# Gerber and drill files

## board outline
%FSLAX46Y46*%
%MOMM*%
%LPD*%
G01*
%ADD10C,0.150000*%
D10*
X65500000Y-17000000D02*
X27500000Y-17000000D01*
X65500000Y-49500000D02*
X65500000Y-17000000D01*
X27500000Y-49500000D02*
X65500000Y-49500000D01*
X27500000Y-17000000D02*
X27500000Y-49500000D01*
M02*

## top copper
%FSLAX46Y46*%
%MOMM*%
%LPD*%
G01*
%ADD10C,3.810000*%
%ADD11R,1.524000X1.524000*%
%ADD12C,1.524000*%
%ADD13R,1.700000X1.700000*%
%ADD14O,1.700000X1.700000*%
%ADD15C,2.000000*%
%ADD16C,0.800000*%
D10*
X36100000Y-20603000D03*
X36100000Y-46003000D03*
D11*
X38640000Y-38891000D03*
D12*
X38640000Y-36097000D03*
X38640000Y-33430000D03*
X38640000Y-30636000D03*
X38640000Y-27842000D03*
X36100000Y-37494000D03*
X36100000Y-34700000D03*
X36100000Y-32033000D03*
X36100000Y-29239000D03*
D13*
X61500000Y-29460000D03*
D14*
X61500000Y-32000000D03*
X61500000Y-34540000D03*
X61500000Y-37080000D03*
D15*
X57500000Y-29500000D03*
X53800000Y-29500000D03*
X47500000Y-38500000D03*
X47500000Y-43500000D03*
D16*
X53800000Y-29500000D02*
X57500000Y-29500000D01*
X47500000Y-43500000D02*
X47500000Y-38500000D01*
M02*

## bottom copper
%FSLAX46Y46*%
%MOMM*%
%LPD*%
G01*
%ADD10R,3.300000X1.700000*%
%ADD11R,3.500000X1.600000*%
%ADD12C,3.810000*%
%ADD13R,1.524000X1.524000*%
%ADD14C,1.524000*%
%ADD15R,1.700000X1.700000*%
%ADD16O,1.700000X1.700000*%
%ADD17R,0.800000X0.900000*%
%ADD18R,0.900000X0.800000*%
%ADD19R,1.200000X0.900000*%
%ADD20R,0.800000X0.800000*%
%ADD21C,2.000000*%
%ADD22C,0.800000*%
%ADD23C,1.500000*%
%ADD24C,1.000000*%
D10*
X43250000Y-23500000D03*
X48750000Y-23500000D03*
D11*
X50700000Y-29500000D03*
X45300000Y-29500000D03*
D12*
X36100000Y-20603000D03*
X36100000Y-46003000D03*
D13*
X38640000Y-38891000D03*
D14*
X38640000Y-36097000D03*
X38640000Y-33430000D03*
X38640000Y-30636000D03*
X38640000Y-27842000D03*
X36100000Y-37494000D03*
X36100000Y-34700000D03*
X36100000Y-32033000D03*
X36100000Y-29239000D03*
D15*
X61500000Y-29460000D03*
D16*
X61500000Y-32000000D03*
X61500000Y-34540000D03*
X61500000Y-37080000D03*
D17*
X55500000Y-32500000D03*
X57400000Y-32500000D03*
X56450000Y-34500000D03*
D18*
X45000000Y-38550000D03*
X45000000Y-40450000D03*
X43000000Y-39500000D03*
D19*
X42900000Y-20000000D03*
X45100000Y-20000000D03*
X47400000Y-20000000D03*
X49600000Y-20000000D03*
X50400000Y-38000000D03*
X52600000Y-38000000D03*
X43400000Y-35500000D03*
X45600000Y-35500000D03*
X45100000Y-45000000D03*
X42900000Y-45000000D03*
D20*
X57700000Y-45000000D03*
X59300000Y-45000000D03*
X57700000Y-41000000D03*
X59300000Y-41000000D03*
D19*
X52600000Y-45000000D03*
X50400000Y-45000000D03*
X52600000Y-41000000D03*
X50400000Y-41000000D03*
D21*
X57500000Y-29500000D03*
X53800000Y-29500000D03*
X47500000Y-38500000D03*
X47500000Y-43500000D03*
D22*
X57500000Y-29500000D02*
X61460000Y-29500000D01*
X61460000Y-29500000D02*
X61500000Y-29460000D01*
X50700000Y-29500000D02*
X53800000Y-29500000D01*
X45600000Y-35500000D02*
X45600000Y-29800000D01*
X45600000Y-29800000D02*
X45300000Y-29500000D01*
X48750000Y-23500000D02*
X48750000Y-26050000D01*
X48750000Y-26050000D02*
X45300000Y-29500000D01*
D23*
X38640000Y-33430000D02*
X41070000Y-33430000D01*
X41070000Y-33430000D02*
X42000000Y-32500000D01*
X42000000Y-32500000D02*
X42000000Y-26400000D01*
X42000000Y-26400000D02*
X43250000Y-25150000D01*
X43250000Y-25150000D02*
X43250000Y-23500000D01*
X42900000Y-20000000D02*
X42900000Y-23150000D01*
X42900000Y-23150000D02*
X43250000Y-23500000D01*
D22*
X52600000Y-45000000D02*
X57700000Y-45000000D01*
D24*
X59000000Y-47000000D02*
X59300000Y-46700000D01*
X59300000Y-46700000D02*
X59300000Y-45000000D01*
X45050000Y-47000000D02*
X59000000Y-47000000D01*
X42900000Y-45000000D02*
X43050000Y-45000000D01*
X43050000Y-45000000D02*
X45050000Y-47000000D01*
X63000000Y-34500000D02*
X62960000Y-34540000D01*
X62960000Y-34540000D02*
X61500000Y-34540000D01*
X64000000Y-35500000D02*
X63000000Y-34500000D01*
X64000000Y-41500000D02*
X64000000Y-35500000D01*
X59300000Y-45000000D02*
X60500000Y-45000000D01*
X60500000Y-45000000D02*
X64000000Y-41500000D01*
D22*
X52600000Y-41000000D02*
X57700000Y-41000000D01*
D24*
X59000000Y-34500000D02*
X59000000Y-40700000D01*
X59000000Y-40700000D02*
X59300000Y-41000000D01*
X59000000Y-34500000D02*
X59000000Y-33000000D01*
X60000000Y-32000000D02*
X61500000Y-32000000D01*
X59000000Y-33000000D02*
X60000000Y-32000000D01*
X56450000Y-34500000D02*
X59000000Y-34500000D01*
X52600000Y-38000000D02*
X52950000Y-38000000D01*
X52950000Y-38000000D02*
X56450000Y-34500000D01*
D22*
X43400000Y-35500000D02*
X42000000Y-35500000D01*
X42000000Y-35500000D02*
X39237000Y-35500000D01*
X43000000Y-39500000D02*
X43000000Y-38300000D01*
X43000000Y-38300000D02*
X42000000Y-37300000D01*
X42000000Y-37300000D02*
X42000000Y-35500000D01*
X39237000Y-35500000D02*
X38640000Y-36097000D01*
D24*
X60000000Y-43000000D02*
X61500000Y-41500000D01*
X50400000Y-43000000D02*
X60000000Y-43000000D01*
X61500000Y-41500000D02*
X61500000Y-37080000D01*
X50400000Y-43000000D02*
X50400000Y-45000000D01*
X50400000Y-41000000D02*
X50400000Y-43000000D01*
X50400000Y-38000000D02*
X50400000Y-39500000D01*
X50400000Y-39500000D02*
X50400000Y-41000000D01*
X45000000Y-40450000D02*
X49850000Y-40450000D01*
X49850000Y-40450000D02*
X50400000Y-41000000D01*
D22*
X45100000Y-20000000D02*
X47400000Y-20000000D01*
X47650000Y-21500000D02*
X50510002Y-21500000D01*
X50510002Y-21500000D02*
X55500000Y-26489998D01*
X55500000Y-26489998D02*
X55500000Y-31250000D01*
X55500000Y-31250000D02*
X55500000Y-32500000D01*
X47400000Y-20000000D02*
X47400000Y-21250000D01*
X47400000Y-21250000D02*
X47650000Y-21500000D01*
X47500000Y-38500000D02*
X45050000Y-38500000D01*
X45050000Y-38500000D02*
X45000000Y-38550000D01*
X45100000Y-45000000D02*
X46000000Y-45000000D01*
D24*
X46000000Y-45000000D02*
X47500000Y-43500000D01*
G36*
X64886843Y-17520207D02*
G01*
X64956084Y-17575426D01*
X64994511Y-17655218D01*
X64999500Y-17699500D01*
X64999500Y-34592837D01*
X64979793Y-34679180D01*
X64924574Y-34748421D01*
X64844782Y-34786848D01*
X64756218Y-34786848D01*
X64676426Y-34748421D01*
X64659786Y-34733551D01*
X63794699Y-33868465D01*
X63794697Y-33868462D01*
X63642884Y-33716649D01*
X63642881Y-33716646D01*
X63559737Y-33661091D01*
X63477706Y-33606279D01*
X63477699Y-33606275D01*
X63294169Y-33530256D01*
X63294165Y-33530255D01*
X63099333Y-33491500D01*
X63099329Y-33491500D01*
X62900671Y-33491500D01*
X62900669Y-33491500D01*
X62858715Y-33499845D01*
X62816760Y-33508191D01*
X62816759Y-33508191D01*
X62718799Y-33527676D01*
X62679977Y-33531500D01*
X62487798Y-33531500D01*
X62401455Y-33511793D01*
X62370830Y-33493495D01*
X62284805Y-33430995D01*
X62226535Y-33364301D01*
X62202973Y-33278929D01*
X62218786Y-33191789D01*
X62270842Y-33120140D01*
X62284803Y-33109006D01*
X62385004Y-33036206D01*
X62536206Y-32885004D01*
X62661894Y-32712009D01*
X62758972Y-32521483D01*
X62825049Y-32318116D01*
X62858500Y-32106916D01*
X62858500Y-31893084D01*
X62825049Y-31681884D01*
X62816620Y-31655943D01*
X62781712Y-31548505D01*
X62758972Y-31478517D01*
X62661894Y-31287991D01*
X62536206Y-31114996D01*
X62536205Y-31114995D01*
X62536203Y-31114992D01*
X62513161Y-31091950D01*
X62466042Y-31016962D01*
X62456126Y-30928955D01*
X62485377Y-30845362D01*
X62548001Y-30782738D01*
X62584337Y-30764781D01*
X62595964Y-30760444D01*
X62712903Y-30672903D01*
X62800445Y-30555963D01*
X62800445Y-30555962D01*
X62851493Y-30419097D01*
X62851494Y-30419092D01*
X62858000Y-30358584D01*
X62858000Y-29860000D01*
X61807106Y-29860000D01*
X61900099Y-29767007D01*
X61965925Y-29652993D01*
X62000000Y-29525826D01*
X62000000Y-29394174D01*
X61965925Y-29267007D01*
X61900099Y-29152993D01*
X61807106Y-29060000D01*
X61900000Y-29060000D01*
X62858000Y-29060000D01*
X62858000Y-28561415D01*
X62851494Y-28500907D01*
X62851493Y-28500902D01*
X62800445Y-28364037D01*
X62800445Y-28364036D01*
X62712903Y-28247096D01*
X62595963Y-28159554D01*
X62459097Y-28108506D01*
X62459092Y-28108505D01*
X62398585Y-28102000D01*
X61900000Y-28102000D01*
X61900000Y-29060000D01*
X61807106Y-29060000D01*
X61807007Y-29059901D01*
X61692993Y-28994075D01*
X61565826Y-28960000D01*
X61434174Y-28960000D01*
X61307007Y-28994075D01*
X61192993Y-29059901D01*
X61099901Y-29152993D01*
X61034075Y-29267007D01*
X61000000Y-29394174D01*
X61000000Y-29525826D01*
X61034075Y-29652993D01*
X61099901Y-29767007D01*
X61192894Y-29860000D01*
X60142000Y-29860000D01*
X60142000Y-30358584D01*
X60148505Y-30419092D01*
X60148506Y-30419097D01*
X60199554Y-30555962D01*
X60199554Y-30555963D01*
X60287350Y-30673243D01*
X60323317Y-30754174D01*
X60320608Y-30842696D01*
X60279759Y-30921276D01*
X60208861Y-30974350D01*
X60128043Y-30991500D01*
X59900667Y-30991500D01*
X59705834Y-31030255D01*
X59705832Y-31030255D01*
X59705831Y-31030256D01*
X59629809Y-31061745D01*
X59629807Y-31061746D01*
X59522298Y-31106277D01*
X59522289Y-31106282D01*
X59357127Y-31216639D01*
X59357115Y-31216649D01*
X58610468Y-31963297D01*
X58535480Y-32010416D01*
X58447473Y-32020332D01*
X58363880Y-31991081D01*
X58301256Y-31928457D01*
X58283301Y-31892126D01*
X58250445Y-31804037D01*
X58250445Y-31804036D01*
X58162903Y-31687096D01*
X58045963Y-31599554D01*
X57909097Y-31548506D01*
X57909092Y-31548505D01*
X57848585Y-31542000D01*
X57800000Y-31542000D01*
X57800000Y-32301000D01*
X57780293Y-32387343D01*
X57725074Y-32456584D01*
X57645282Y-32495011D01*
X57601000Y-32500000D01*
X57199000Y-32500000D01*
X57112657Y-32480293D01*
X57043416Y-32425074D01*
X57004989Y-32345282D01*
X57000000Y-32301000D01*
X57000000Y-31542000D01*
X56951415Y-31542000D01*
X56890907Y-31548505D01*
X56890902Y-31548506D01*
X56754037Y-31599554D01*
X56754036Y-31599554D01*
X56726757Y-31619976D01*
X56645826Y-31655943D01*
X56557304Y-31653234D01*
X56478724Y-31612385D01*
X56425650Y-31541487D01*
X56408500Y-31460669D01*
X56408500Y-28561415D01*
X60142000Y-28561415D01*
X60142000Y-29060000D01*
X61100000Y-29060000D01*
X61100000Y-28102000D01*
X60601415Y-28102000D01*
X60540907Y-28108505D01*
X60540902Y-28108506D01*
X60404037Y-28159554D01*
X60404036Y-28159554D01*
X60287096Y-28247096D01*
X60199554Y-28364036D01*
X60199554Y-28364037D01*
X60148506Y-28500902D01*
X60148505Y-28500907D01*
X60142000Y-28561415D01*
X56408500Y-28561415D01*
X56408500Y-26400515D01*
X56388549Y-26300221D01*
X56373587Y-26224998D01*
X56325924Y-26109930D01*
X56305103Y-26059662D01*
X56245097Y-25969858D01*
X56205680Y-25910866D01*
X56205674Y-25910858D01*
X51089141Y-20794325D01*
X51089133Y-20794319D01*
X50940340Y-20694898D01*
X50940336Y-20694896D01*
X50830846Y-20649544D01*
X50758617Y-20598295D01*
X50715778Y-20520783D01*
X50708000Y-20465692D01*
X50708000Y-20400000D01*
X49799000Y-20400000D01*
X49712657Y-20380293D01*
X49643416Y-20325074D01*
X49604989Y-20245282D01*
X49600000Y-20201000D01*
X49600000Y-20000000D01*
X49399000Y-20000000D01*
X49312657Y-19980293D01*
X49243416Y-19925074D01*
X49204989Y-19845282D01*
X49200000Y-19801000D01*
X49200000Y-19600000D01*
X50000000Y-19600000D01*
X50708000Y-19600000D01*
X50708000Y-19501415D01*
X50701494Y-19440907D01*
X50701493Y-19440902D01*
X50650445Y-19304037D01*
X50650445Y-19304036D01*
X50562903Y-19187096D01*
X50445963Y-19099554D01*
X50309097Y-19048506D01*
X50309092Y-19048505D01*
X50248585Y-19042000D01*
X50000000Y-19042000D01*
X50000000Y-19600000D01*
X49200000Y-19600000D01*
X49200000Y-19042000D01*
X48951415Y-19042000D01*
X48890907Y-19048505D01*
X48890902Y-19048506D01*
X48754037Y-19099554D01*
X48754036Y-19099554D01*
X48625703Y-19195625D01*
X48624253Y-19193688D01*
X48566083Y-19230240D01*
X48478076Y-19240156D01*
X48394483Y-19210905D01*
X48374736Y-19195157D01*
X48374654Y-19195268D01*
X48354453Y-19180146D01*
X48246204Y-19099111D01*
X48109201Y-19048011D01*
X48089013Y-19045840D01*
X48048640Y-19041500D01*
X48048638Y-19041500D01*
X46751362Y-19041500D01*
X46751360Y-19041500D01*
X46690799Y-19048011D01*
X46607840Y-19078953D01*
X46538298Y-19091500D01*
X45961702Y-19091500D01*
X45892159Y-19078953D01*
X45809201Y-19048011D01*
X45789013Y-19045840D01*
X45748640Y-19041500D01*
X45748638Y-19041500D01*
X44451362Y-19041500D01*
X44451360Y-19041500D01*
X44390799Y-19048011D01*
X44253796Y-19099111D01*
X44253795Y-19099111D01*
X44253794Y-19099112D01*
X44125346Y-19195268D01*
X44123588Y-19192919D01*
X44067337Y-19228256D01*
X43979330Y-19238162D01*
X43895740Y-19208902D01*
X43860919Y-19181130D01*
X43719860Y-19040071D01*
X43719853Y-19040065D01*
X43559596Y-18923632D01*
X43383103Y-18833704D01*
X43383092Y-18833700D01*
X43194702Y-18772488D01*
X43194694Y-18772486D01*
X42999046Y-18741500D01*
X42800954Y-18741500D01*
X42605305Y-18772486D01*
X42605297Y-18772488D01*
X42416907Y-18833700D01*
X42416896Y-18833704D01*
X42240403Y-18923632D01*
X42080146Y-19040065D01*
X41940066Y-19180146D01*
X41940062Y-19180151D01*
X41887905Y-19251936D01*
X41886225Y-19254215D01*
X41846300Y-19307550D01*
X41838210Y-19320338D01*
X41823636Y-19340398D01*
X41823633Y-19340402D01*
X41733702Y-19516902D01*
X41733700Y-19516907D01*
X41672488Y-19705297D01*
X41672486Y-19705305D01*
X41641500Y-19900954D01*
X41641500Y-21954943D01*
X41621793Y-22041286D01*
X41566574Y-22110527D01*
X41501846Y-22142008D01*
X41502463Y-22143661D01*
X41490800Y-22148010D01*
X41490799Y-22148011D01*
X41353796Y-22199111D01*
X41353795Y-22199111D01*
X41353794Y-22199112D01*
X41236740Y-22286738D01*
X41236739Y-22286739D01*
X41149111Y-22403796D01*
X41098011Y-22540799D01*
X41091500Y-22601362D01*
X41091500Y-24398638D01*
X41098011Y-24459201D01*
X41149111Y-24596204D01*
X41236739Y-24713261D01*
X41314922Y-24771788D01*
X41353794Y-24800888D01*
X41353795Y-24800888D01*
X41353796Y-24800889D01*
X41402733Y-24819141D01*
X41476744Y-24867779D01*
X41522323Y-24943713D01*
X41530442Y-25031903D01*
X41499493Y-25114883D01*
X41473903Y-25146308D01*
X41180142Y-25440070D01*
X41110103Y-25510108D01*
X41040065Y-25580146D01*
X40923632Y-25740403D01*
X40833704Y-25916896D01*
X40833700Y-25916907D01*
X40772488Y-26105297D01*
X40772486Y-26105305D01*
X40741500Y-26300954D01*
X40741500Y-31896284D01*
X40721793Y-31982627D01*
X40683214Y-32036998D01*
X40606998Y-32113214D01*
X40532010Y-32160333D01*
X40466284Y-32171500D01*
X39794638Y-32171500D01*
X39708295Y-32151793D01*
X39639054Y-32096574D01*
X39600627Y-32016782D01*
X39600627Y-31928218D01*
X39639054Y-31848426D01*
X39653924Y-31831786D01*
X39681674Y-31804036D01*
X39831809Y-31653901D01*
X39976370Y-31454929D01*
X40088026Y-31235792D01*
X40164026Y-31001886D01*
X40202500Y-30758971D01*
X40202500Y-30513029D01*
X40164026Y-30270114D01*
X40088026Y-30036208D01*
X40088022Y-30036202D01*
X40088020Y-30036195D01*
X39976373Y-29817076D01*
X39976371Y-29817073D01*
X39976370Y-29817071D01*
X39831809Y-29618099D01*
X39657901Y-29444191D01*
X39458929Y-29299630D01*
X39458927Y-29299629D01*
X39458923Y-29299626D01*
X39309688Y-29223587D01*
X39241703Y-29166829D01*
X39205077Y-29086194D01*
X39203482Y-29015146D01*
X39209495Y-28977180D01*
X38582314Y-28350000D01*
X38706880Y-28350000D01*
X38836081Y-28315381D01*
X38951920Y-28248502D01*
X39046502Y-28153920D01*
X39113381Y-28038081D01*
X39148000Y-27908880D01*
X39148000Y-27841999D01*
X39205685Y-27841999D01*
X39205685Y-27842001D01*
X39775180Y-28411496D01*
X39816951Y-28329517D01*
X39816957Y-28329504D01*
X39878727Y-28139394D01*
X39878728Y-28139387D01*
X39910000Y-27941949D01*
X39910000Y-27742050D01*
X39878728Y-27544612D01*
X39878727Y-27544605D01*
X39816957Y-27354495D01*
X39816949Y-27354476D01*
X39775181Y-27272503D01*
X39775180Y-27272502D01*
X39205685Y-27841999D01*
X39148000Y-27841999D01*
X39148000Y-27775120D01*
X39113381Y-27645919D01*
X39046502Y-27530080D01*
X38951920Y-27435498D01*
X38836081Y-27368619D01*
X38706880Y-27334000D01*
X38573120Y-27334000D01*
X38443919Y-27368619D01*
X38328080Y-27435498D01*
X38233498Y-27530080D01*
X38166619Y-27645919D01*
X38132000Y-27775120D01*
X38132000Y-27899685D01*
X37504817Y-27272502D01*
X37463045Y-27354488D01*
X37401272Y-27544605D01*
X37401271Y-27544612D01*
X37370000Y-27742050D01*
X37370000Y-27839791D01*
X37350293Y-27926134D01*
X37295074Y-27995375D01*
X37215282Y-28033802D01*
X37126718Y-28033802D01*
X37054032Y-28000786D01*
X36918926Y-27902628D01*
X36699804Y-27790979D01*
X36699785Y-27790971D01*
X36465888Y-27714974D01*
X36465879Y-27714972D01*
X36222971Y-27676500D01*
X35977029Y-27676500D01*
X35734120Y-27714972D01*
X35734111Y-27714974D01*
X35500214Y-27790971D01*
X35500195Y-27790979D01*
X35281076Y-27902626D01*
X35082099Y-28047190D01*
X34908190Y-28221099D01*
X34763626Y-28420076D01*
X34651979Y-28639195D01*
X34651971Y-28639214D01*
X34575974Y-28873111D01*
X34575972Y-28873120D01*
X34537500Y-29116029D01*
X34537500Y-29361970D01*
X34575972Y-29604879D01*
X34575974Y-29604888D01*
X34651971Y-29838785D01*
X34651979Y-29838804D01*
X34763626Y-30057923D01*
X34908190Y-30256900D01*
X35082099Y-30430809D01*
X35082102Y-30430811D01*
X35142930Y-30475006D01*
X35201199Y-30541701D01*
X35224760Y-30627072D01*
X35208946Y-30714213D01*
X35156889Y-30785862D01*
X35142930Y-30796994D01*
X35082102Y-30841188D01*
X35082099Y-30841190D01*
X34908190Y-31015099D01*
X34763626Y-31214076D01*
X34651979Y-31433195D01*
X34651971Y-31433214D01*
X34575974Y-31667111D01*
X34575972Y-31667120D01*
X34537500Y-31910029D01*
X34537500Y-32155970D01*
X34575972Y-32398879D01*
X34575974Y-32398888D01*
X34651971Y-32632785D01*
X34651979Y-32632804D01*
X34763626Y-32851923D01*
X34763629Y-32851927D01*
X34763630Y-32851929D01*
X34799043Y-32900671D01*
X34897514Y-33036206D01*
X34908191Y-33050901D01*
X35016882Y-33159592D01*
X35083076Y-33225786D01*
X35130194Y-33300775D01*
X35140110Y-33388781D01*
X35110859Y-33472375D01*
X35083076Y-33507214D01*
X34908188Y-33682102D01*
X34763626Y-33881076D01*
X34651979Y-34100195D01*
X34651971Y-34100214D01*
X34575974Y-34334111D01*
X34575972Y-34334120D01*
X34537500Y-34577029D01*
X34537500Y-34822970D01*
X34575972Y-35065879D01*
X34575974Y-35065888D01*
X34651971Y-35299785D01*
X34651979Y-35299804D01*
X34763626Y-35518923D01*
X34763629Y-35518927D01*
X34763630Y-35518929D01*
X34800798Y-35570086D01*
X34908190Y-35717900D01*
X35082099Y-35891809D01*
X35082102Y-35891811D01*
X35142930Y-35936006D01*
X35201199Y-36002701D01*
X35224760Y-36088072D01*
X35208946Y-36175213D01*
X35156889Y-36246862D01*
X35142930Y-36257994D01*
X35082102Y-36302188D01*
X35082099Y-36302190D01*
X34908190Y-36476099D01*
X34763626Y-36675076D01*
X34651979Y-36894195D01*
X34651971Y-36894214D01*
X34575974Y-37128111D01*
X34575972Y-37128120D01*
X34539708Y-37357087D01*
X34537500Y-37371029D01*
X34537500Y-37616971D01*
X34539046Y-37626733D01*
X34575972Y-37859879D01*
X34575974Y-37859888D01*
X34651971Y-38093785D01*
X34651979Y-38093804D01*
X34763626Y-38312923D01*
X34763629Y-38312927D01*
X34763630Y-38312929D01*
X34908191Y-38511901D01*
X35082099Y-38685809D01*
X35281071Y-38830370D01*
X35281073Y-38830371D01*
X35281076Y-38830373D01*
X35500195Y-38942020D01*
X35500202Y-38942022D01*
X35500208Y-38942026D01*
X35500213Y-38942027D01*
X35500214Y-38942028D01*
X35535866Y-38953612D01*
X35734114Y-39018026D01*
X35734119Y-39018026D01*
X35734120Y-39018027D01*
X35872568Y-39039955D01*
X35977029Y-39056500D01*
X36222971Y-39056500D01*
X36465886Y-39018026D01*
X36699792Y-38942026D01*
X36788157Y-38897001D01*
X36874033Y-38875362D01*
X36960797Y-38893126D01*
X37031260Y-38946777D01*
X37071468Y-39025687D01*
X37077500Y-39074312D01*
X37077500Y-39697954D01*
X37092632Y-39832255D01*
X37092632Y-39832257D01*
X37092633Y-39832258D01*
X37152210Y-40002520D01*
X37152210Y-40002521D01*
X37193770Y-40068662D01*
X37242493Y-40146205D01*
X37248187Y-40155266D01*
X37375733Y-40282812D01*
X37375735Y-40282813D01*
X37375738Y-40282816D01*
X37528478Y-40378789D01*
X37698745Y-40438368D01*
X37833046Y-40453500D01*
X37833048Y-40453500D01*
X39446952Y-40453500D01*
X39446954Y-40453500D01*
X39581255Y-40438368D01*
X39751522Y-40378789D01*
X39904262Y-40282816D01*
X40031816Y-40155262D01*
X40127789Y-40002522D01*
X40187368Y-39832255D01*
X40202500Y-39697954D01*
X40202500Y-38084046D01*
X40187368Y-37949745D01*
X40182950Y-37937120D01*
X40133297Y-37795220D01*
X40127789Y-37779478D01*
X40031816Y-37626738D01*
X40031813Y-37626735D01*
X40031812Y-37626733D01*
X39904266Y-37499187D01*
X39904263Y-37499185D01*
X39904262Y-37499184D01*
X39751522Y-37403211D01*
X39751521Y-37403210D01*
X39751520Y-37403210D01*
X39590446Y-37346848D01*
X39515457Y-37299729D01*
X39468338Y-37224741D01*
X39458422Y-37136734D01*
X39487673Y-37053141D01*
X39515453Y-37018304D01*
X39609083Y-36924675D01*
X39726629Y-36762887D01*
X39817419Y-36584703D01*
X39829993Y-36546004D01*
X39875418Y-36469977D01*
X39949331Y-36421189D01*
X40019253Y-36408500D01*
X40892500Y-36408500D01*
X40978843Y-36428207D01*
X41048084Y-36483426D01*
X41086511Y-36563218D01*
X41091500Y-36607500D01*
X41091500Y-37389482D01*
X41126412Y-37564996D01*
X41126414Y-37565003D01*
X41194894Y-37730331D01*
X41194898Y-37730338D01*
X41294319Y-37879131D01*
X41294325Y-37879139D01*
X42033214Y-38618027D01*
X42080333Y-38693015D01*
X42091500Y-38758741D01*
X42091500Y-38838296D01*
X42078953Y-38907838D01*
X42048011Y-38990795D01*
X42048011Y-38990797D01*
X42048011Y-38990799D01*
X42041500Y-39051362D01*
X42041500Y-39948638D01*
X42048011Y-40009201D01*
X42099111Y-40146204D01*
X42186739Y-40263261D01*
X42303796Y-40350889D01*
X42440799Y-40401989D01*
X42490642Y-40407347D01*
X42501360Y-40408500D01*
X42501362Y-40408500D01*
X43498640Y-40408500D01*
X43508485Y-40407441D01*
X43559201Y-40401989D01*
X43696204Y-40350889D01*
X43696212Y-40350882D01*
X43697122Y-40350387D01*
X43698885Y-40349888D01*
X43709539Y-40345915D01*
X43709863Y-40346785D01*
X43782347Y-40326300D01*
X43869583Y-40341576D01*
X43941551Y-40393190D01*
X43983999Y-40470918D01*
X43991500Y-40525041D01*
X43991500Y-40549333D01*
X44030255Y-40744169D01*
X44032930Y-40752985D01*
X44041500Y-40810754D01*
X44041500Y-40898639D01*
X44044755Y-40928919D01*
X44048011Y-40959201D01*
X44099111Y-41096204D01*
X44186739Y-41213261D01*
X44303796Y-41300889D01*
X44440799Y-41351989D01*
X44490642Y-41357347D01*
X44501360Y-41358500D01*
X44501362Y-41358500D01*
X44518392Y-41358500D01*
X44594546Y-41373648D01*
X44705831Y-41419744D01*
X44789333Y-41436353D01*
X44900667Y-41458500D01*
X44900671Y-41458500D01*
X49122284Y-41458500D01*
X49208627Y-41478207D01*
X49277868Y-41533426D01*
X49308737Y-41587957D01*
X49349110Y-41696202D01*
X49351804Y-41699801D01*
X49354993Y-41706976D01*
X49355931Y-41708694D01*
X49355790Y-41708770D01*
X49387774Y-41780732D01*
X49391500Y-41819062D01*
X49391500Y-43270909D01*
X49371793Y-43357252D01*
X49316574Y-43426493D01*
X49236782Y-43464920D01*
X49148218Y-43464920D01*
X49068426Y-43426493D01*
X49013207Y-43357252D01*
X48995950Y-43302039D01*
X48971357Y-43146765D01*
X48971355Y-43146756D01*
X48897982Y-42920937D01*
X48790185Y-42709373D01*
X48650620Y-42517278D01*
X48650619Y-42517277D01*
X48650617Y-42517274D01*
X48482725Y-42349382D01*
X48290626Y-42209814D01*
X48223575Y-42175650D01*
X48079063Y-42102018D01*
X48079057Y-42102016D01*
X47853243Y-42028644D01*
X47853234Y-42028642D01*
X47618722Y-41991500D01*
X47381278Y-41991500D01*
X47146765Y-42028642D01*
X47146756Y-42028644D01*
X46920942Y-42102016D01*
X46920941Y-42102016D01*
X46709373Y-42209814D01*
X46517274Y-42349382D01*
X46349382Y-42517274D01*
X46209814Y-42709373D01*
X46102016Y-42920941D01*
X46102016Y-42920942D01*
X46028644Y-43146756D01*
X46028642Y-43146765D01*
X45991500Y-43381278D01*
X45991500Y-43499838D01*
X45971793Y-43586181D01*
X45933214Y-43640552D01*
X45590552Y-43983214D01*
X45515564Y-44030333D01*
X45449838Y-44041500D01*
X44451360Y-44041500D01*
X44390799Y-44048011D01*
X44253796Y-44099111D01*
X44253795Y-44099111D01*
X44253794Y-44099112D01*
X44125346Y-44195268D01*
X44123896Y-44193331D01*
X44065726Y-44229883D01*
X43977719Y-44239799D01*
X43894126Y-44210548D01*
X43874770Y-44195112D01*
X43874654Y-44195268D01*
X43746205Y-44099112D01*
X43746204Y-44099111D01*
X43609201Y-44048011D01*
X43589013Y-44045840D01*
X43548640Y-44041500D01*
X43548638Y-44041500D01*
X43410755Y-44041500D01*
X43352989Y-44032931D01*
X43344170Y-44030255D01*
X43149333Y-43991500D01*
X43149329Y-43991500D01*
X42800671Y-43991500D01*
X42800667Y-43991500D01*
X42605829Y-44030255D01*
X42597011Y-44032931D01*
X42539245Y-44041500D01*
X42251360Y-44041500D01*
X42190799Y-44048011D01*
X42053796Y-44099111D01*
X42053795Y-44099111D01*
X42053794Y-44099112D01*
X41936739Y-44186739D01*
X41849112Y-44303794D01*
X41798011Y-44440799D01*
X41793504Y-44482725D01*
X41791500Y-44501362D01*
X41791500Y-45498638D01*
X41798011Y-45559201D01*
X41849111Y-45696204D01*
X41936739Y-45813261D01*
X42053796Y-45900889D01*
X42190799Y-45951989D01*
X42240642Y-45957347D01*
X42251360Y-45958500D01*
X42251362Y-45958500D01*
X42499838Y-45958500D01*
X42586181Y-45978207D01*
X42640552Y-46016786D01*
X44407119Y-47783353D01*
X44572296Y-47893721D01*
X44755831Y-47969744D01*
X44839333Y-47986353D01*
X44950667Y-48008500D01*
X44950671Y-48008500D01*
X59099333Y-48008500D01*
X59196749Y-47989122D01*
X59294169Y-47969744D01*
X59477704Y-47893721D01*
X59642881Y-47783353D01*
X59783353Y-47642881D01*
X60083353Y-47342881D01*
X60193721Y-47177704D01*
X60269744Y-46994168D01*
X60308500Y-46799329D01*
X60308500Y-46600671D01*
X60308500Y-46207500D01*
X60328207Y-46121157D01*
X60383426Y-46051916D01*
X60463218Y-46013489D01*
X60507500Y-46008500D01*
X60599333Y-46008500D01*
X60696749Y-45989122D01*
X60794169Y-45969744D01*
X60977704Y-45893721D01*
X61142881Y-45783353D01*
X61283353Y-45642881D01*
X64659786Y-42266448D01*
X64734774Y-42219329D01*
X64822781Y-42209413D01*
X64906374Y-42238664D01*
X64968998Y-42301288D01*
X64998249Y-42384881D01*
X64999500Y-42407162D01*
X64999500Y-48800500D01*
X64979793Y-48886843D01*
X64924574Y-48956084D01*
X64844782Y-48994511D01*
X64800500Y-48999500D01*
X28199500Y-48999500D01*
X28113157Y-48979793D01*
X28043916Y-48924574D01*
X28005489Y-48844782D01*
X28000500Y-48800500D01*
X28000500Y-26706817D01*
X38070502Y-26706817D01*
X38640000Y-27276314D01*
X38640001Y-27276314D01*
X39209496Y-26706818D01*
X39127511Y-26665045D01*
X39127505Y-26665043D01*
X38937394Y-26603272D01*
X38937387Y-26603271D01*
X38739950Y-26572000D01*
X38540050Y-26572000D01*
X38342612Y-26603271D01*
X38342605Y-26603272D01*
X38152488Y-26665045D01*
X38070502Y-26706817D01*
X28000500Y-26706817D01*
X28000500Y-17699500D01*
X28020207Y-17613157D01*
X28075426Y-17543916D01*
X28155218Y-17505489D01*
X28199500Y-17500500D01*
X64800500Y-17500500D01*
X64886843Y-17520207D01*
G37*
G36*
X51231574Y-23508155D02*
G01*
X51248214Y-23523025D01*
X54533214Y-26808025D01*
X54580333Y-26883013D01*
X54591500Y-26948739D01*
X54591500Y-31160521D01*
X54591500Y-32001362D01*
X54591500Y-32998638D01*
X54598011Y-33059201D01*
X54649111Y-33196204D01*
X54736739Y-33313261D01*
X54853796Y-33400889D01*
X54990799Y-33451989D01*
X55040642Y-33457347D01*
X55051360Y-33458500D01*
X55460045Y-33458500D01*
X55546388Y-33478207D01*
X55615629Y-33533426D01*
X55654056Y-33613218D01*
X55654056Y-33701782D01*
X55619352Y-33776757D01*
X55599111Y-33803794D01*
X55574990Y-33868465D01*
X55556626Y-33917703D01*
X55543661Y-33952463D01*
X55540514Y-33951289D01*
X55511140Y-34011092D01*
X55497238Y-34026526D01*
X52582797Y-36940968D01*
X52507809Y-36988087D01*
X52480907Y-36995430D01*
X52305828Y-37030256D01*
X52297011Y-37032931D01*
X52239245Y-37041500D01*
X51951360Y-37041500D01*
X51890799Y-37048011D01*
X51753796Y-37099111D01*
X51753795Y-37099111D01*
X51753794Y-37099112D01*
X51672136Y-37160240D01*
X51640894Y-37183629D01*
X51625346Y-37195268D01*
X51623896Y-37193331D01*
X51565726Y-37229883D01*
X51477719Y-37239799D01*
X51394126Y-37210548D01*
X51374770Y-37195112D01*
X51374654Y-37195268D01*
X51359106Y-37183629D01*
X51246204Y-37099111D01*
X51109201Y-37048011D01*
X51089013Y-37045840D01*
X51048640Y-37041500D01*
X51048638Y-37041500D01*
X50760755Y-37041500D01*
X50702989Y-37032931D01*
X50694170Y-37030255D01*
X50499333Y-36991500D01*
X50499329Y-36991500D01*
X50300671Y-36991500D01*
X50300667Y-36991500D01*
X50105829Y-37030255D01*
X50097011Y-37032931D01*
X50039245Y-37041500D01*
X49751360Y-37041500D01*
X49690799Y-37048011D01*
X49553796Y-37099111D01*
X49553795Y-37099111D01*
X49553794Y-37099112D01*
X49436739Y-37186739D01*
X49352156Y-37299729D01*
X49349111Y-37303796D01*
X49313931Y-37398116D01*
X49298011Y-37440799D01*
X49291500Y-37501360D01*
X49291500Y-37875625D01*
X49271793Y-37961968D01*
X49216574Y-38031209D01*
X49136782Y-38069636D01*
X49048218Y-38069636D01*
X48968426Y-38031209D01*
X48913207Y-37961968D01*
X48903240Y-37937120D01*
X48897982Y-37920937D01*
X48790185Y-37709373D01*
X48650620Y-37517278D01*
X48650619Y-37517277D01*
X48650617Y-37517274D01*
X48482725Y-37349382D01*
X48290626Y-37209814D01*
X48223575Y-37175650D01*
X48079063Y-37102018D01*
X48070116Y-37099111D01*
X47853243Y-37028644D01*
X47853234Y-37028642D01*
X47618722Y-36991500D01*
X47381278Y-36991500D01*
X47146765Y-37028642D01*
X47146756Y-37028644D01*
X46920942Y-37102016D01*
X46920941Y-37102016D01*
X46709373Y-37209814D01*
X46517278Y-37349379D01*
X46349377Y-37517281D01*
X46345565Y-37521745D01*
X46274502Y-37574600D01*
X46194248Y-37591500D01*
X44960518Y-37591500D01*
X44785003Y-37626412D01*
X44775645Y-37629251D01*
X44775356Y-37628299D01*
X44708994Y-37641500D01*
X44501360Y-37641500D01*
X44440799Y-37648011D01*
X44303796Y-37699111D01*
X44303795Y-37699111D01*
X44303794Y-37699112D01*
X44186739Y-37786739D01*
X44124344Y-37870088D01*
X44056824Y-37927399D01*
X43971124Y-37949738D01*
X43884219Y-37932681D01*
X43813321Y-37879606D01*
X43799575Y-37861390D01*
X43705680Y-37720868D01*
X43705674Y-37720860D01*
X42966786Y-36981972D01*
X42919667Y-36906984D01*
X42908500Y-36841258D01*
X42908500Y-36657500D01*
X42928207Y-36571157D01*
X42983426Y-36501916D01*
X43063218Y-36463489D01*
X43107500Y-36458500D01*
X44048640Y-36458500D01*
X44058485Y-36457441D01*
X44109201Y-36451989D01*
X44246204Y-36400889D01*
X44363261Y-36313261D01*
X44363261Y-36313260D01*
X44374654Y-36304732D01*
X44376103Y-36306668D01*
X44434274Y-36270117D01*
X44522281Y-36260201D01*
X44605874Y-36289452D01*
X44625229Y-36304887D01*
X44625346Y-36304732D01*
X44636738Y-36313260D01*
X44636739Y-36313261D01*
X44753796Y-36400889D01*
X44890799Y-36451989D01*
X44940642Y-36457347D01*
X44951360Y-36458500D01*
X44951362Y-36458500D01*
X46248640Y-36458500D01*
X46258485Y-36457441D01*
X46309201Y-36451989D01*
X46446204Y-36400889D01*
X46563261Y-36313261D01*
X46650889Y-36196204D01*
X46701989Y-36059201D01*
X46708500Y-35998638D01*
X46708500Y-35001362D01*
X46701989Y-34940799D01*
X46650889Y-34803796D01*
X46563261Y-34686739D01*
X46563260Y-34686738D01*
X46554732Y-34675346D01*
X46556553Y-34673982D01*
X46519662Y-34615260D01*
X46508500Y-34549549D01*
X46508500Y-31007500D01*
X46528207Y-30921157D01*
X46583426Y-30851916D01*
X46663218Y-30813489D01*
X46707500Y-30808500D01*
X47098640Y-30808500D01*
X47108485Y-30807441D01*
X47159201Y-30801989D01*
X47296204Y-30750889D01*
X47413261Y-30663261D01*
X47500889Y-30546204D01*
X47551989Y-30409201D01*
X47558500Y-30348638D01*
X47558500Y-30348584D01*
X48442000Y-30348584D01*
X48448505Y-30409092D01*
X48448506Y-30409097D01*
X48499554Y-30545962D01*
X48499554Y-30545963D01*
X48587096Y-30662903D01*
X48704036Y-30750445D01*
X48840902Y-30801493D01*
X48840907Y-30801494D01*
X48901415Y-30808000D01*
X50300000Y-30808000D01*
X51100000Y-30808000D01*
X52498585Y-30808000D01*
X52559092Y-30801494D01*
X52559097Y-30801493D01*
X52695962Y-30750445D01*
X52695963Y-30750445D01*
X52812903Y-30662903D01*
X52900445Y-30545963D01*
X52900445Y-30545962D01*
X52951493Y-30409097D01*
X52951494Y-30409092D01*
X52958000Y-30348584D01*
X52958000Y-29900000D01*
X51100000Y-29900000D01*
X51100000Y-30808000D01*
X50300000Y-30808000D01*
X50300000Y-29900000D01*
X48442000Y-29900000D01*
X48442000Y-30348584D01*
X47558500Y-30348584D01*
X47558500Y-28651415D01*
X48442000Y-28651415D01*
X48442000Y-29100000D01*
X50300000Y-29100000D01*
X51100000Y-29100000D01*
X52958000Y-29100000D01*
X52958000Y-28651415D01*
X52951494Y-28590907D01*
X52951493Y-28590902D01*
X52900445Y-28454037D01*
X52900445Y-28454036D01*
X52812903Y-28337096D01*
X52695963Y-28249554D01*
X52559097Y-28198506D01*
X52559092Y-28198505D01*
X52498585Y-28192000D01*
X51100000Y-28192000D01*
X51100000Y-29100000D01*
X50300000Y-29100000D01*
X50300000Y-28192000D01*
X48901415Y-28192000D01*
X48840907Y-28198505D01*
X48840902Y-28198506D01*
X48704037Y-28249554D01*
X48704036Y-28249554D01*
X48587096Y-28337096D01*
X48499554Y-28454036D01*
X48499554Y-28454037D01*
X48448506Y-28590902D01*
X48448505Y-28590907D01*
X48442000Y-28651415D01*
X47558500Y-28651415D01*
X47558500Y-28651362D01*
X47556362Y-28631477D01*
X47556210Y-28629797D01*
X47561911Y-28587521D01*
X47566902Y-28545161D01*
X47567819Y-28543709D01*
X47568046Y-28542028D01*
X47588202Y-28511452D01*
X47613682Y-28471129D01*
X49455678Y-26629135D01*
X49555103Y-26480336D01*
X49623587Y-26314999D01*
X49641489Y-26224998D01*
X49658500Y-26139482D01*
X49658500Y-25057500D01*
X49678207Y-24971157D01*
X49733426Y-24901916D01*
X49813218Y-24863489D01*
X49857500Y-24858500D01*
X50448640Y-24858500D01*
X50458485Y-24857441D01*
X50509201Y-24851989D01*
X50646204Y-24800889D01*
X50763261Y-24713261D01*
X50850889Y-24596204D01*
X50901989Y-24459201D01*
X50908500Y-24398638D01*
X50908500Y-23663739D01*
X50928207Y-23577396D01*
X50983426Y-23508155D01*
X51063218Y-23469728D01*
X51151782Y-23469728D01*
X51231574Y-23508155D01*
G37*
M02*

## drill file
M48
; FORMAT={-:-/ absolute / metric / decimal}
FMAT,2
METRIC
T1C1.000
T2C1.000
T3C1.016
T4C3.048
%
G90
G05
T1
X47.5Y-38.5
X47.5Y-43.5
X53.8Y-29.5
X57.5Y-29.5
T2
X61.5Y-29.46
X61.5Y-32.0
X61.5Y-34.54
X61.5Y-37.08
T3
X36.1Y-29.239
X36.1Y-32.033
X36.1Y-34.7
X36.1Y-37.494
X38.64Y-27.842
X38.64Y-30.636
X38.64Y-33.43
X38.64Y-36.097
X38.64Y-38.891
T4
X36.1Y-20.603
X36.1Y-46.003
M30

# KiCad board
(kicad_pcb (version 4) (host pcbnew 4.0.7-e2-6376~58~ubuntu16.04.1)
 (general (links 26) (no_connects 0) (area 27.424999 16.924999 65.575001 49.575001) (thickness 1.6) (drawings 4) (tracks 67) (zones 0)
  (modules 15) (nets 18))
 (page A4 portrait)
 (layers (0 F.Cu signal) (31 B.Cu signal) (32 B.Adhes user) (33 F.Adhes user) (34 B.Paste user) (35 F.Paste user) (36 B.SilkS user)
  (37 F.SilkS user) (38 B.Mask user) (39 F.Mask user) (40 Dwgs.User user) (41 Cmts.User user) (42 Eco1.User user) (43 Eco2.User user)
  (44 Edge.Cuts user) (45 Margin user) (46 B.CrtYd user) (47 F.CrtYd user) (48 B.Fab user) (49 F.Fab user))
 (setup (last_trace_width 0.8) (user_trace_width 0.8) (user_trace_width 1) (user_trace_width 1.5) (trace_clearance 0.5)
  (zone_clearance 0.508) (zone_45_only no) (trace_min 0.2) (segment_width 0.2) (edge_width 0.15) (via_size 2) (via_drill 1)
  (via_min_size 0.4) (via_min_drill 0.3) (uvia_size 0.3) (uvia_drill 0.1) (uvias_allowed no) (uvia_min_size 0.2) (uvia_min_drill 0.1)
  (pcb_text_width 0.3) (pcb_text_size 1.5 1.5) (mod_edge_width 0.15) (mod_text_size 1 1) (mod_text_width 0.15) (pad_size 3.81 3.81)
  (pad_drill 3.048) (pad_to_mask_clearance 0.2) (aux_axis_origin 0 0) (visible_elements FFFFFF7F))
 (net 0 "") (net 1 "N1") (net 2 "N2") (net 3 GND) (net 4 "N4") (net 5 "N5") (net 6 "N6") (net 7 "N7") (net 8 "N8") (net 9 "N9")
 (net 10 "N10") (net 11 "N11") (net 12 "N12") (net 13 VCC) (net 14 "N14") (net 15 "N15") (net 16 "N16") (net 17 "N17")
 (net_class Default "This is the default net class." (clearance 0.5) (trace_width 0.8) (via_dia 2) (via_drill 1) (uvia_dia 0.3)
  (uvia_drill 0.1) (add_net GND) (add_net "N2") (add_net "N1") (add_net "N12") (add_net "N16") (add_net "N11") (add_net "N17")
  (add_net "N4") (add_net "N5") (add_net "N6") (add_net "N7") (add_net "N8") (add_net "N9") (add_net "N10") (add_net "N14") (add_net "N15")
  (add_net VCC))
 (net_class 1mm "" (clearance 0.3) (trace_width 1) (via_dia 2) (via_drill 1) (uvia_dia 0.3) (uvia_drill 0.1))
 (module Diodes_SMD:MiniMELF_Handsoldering (layer B.Cu) (at 46 23.5)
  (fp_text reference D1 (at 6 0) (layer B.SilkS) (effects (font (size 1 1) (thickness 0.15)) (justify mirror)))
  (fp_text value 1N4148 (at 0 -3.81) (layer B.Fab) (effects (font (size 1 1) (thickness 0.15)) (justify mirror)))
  (pad 1 smd rect (at -2.75 0) (size 3.3 1.7) (layers B.Cu B.Paste B.Mask) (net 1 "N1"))
  (pad 2 smd rect (at 2.75 0) (size 3.3 1.7) (layers B.Cu B.Paste B.Mask) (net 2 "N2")))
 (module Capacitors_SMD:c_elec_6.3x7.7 (layer B.Cu) (at 48 29.5 180)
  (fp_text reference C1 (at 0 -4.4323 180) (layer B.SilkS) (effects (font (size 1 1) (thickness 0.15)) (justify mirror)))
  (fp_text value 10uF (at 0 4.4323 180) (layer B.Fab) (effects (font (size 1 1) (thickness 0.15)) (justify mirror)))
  (pad 1 smd rect (at -2.7 0) (size 3.5 1.6) (layers B.Cu B.Paste B.Mask) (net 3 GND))
  (pad 2 smd rect (at 2.7 0) (size 3.5 1.6) (layers B.Cu B.Paste B.Mask) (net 2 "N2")))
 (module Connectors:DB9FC (layer F.Cu) (at 37.37 33.43 90)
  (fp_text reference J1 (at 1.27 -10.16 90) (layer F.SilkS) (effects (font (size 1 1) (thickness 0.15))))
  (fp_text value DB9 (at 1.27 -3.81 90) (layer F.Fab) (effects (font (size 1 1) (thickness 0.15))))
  (pad "" thru_hole circle (at 12.827 -1.27 90) (size 3.81 3.81) (drill 3.048) (layers *.Cu *.Mask) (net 3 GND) (zone_connect 2))
  (pad "" thru_hole circle (at -12.573 -1.27 90) (size 3.81 3.81) (drill 3.048) (layers *.Cu *.Mask) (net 3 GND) (zone_connect 2))
  (pad 1 thru_hole rect (at -5.461 1.27 90) (size 1.524 1.524) (drill 1.016) (layers *.Cu *.Mask) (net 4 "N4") (clearance 0.8))
  (pad 2 thru_hole circle (at -2.667 1.27 90) (size 1.524 1.524) (drill 1.016) (layers *.Cu *.Mask) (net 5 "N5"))
  (pad 3 thru_hole circle (at 0 1.27 90) (size 1.524 1.524) (drill 1.016) (layers *.Cu *.Mask) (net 1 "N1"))
  (pad 4 thru_hole circle (at 2.794 1.27 90) (size 1.524 1.524) (drill 1.016) (layers *.Cu *.Mask) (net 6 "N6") (clearance 0.8))
  (pad 5 thru_hole circle (at 5.588 1.27 90) (size 1.524 1.524) (drill 1.016) (layers *.Cu *.Mask) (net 3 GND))
  (pad 6 thru_hole circle (at -4.064 -1.27 90) (size 1.524 1.524) (drill 1.016) (layers *.Cu *.Mask) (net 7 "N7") (clearance 0.8))
  (pad 7 thru_hole circle (at -1.27 -1.27 90) (size 1.524 1.524) (drill 1.016) (layers *.Cu *.Mask) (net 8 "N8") (clearance 0.8))
  (pad 8 thru_hole circle (at 1.397 -1.27 90) (size 1.524 1.524) (drill 1.016) (layers *.Cu *.Mask) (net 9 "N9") (clearance 0.8))
  (pad 9 thru_hole circle (at 4.191 -1.27 90) (size 1.524 1.524) (drill 1.016) (layers *.Cu *.Mask) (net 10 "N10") (clearance 0.8)))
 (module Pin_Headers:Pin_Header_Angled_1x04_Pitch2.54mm (layer F.Cu) (at 61.5 29.46)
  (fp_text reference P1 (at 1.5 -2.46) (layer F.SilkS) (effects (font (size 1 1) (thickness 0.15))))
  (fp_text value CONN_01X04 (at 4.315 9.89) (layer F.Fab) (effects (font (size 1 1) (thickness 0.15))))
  (pad 1 thru_hole rect (at 0 0) (size 1.7 1.7) (drill 1) (layers *.Cu *.Mask) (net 3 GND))
  (pad 2 thru_hole oval (at 0 2.54) (size 1.7 1.7) (drill 1) (layers *.Cu *.Mask) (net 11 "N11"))
  (pad 3 thru_hole oval (at 0 5.08) (size 1.7 1.7) (drill 1) (layers *.Cu *.Mask) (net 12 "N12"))
  (pad 4 thru_hole oval (at 0 7.62) (size 1.7 1.7) (drill 1) (layers *.Cu *.Mask) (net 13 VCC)))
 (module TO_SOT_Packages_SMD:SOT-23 (layer B.Cu) (at 56.45 33.5 270)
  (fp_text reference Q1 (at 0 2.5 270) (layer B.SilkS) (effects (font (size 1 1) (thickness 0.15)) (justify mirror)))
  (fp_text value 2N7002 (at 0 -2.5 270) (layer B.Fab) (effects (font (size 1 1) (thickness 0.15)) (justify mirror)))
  (pad 1 smd rect (at -1 0.95 270) (size 0.9 0.8) (layers B.Cu B.Paste B.Mask) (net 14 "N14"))
  (pad 2 smd rect (at -1 -0.95 270) (size 0.9 0.8) (layers B.Cu B.Paste B.Mask) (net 3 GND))
  (pad 3 smd rect (at 1 0 270) (size 0.9 0.8) (layers B.Cu B.Paste B.Mask) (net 11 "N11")))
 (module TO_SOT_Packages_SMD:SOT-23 (layer B.Cu) (at 44 39.5 180)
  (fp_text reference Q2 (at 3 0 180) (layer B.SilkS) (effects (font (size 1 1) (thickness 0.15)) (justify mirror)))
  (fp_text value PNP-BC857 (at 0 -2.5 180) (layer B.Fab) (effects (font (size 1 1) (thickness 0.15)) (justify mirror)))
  (pad 1 smd rect (at -1 0.95 180) (size 0.9 0.8) (layers B.Cu B.Paste B.Mask) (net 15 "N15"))
  (pad 2 smd rect (at -1 -0.95 180) (size 0.9 0.8) (layers B.Cu B.Paste B.Mask) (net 13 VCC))
  (pad 3 smd rect (at 1 0 180) (size 0.9 0.8) (layers B.Cu B.Paste B.Mask) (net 5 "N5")))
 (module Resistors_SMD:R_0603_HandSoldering (layer B.Cu) (at 44 20)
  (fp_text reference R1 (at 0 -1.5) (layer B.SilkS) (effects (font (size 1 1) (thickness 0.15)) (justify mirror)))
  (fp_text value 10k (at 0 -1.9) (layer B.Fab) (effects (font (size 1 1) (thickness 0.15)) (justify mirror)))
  (pad 1 smd rect (at -1.1 0) (size 1.2 0.9) (layers B.Cu B.Paste B.Mask) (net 1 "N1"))
  (pad 2 smd rect (at 1.1 0) (size 1.2 0.9) (layers B.Cu B.Paste B.Mask) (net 14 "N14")))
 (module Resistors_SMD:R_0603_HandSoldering (layer B.Cu) (at 48.5 20)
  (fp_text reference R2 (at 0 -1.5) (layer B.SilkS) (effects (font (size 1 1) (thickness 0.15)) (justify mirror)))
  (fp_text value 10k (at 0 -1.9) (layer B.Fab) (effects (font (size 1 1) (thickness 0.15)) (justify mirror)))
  (pad 1 smd rect (at -1.1 0) (size 1.2 0.9) (layers B.Cu B.Paste B.Mask) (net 14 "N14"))
  (pad 2 smd rect (at 1.1 0) (size 1.2 0.9) (layers B.Cu B.Paste B.Mask) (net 3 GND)))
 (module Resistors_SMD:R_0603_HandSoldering (layer B.Cu) (at 51.5 38)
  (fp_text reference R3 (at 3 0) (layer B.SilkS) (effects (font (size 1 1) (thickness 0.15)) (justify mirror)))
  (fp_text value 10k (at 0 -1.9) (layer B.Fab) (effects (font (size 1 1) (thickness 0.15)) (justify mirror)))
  (pad 1 smd rect (at -1.1 0) (size 1.2 0.9) (layers B.Cu B.Paste B.Mask) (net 13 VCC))
  (pad 2 smd rect (at 1.1 0) (size 1.2 0.9) (layers B.Cu B.Paste B.Mask) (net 11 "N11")))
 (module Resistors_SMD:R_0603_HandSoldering (layer B.Cu) (at 44.5 35.5)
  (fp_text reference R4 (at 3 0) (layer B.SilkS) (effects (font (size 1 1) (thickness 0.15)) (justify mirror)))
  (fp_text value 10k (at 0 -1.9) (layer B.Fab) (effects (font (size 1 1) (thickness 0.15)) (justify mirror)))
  (pad 1 smd rect (at -1.1 0) (size 1.2 0.9) (layers B.Cu B.Paste B.Mask) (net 5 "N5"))
  (pad 2 smd rect (at 1.1 0) (size 1.2 0.9) (layers B.Cu B.Paste B.Mask) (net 2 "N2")))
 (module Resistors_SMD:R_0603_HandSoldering (layer B.Cu) (at 44 45 180)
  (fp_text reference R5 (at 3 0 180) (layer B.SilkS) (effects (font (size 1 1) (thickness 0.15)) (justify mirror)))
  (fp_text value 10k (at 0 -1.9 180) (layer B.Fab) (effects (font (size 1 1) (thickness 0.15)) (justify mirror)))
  (pad 1 smd rect (at -1.1 0 180) (size 1.2 0.9) (layers B.Cu B.Paste B.Mask) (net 15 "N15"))
  (pad 2 smd rect (at 1.1 0 180) (size 1.2 0.9) (layers B.Cu B.Paste B.Mask) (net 12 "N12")))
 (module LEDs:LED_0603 (layer B.Cu) (at 58.5 45 180)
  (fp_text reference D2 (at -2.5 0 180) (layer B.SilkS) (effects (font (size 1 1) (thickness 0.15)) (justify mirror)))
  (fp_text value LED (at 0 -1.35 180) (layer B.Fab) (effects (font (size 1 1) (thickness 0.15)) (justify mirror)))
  (pad 2 smd rect (at 0.8 0) (size 0.8 0.8) (layers B.Cu B.Paste B.Mask) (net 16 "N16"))
  (pad 1 smd rect (at -0.8 0) (size 0.8 0.8) (layers B.Cu B.Paste B.Mask) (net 12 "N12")))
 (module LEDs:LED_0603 (layer B.Cu) (at 58.5 41 180)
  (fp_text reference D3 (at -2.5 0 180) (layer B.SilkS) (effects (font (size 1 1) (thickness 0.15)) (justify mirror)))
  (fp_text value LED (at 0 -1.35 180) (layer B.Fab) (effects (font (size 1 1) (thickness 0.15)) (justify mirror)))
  (pad 2 smd rect (at 0.8 0) (size 0.8 0.8) (layers B.Cu B.Paste B.Mask) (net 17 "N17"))
  (pad 1 smd rect (at -0.8 0) (size 0.8 0.8) (layers B.Cu B.Paste B.Mask) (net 11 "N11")))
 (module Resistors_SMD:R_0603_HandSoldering (layer B.Cu) (at 51.5 45 180)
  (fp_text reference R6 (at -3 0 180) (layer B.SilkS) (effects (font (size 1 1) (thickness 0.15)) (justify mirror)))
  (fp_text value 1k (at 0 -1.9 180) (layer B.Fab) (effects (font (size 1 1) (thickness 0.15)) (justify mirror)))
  (pad 1 smd rect (at -1.1 0 180) (size 1.2 0.9) (layers B.Cu B.Paste B.Mask) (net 16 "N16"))
  (pad 2 smd rect (at 1.1 0 180) (size 1.2 0.9) (layers B.Cu B.Paste B.Mask) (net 13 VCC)))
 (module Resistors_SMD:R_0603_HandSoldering (layer B.Cu) (at 51.5 41 180)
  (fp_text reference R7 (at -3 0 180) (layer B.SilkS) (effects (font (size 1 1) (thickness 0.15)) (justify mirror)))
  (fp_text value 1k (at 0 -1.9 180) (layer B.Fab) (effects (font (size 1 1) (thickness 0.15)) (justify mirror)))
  (pad 1 smd rect (at -1.1 0 180) (size 1.2 0.9) (layers B.Cu B.Paste B.Mask) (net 17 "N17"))
  (pad 2 smd rect (at 1.1 0 180) (size 1.2 0.9) (layers B.Cu B.Paste B.Mask) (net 13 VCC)))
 (gr_line (start 65.5 17) (end 27.5 17) (layer Edge.Cuts) (width 0.15))
 (gr_line (start 65.5 49.5) (end 65.5 17) (layer Edge.Cuts) (width 0.15))
 (gr_line (start 27.5 49.5) (end 65.5 49.5) (layer Edge.Cuts) (width 0.15))
 (gr_line (start 27.5 17) (end 27.5 49.5) (layer Edge.Cuts) (width 0.15))
 (segment (start 57.5 29.5) (end 61.46 29.5) (width 0.8) (layer B.Cu) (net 3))
 (segment (start 61.46 29.5) (end 61.5 29.46) (width 0.8) (layer B.Cu) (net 3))
 (segment (start 53.8 29.5) (end 57.5 29.5) (width 0.8) (layer F.Cu) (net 3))
 (via (at 57.5 29.5) (size 2) (drill 1) (layers F.Cu B.Cu) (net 3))
 (segment (start 50.7 29.5) (end 53.8 29.5) (width 0.8) (layer B.Cu) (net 3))
 (via (at 53.8 29.5) (size 2) (drill 1) (layers F.Cu B.Cu) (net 3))
 (segment (start 45.6 35.5) (end 45.6 29.8) (width 0.8) (layer B.Cu) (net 2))
 (segment (start 45.6 29.8) (end 45.3 29.5) (width 0.8) (layer B.Cu) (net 2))
 (segment (start 48.75 23.5) (end 48.75 26.05) (width 0.8) (layer B.Cu) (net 2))
 (segment (start 48.75 26.05) (end 45.3 29.5) (width 0.8) (layer B.Cu) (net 2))
 (segment (start 38.64 33.43) (end 41.07 33.43) (width 1.5) (layer B.Cu) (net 1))
 (segment (start 41.07 33.43) (end 42 32.5) (width 1.5) (layer B.Cu) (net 1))
 (segment (start 42 32.5) (end 42 26.4) (width 1.5) (layer B.Cu) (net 1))
 (segment (start 42 26.4) (end 43.25 25.15) (width 1.5) (layer B.Cu) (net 1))
 (segment (start 43.25 25.15) (end 43.25 23.5) (width 1.5) (layer B.Cu) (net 1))
 (segment (start 42.9 20) (end 42.9 23.15) (width 1.5) (layer B.Cu) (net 1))
 (segment (start 42.9 23.15) (end 43.25 23.5) (width 1.5) (layer B.Cu) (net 1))
 (segment (start 52.6 45) (end 57.7 45) (width 0.8) (layer B.Cu) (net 16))
 (segment (start 59 47) (end 59.3 46.7) (width 1) (layer B.Cu) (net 12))
 (segment (start 59.3 46.7) (end 59.3 45) (width 1) (layer B.Cu) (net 12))
 (segment (start 45.05 47) (end 59 47) (width 1) (layer B.Cu) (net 12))
 (segment (start 42.9 45) (end 43.05 45) (width 1) (layer B.Cu) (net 12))
 (segment (start 43.05 45) (end 45.05 47) (width 1) (layer B.Cu) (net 12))
 (segment (start 63 34.5) (end 62.96 34.54) (width 1) (layer B.Cu) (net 12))
 (segment (start 62.96 34.54) (end 61.5 34.54) (width 1) (layer B.Cu) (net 12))
 (segment (start 64 35.5) (end 63 34.5) (width 1) (layer B.Cu) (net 12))
 (segment (start 64 41.5) (end 64 35.5) (width 1) (layer B.Cu) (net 12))
 (segment (start 59.3 45) (end 60.5 45) (width 1) (layer B.Cu) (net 12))
 (segment (start 60.5 45) (end 64 41.5) (width 1) (layer B.Cu) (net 12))
 (segment (start 52.6 41) (end 57.7 41) (width 0.8) (layer B.Cu) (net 17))
 (segment (start 59 34.5) (end 59 40.7) (width 1) (layer B.Cu) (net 11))
 (segment (start 59 40.7) (end 59.3 41) (width 1) (layer B.Cu) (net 11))
 (segment (start 59 34.5) (end 59 33) (width 1) (layer B.Cu) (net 11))
 (segment (start 60 32) (end 61.5 32) (width 1) (layer B.Cu) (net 11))
 (segment (start 59 33) (end 60 32) (width 1) (layer B.Cu) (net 11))
 (segment (start 56.45 34.5) (end 59 34.5) (width 1) (layer B.Cu) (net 11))
 (segment (start 52.6 38) (end 52.95 38) (width 1) (layer B.Cu) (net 11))
 (segment (start 52.95 38) (end 56.45 34.5) (width 1) (layer B.Cu) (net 11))
 (segment (start 43.4 35.5) (end 42 35.5) (width 0.8) (layer B.Cu) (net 5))
 (segment (start 42 35.5) (end 39.237 35.5) (width 0.8) (layer B.Cu) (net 5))
 (segment (start 43 39.5) (end 43 38.3) (width 0.8) (layer B.Cu) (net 5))
 (segment (start 43 38.3) (end 42 37.3) (width 0.8) (layer B.Cu) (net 5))
 (segment (start 42 37.3) (end 42 35.5) (width 0.8) (layer B.Cu) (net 5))
 (segment (start 39.237 35.5) (end 38.64 36.097) (width 0.8) (layer B.Cu) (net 5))
 (segment (start 60 43) (end 61.5 41.5) (width 1) (layer B.Cu) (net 13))
 (segment (start 50.4 43) (end 60 43) (width 1) (layer B.Cu) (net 13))
 (segment (start 61.5 41.5) (end 61.5 37.08) (width 1) (layer B.Cu) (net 13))
 (segment (start 50.4 43) (end 50.4 45) (width 1) (layer B.Cu) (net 13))
 (segment (start 50.4 41) (end 50.4 43) (width 1) (layer B.Cu) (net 13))
 (segment (start 50.4 38) (end 50.4 39.5) (width 1) (layer B.Cu) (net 13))
 (segment (start 50.4 39.5) (end 50.4 41) (width 1) (layer B.Cu) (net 13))
 (segment (start 45 40.45) (end 49.85 40.45) (width 1) (layer B.Cu) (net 13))
 (segment (start 49.85 40.45) (end 50.4 41) (width 1) (layer B.Cu) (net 13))
 (segment (start 45.1 20) (end 47.4 20) (width 0.8) (layer B.Cu) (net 14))
 (segment (start 47.65 21.5) (end 50.510002 21.5) (width 0.8) (layer B.Cu) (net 14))
 (segment (start 50.510002 21.5) (end 55.5 26.489998) (width 0.8) (layer B.Cu) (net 14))
 (segment (start 55.5 26.489998) (end 55.5 31.25) (width 0.8) (layer B.Cu) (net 14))
 (segment (start 55.5 31.25) (end 55.5 32.5) (width 0.8) (layer B.Cu) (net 14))
 (segment (start 47.4 20) (end 47.4 21.25) (width 0.8) (layer B.Cu) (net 14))
 (segment (start 47.4 21.25) (end 47.65 21.5) (width 0.8) (layer B.Cu) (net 14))
 (segment (start 47.5 38.5) (end 45.05 38.5) (width 0.8) (layer B.Cu) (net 15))
 (segment (start 45.05 38.5) (end 45 38.55) (width 0.8) (layer B.Cu) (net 15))
 (segment (start 47.5 43.5) (end 47.5 38.5) (width 0.8) (layer F.Cu) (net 15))
 (via (at 47.5 38.5) (size 2) (drill 1) (layers F.Cu B.Cu) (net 15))
 (segment (start 45.1 45) (end 46 45) (width 0.8) (layer B.Cu) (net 15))
 (segment (start 46 45) (end 47.5 43.5) (width 1) (layer B.Cu) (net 15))
 (via (at 47.5 43.5) (size 2) (drill 1) (layers F.Cu B.Cu) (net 15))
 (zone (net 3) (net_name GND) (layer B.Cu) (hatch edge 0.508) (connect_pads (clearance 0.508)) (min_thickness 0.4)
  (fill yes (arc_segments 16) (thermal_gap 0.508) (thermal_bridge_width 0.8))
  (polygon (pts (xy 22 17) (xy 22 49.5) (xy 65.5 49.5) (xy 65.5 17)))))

